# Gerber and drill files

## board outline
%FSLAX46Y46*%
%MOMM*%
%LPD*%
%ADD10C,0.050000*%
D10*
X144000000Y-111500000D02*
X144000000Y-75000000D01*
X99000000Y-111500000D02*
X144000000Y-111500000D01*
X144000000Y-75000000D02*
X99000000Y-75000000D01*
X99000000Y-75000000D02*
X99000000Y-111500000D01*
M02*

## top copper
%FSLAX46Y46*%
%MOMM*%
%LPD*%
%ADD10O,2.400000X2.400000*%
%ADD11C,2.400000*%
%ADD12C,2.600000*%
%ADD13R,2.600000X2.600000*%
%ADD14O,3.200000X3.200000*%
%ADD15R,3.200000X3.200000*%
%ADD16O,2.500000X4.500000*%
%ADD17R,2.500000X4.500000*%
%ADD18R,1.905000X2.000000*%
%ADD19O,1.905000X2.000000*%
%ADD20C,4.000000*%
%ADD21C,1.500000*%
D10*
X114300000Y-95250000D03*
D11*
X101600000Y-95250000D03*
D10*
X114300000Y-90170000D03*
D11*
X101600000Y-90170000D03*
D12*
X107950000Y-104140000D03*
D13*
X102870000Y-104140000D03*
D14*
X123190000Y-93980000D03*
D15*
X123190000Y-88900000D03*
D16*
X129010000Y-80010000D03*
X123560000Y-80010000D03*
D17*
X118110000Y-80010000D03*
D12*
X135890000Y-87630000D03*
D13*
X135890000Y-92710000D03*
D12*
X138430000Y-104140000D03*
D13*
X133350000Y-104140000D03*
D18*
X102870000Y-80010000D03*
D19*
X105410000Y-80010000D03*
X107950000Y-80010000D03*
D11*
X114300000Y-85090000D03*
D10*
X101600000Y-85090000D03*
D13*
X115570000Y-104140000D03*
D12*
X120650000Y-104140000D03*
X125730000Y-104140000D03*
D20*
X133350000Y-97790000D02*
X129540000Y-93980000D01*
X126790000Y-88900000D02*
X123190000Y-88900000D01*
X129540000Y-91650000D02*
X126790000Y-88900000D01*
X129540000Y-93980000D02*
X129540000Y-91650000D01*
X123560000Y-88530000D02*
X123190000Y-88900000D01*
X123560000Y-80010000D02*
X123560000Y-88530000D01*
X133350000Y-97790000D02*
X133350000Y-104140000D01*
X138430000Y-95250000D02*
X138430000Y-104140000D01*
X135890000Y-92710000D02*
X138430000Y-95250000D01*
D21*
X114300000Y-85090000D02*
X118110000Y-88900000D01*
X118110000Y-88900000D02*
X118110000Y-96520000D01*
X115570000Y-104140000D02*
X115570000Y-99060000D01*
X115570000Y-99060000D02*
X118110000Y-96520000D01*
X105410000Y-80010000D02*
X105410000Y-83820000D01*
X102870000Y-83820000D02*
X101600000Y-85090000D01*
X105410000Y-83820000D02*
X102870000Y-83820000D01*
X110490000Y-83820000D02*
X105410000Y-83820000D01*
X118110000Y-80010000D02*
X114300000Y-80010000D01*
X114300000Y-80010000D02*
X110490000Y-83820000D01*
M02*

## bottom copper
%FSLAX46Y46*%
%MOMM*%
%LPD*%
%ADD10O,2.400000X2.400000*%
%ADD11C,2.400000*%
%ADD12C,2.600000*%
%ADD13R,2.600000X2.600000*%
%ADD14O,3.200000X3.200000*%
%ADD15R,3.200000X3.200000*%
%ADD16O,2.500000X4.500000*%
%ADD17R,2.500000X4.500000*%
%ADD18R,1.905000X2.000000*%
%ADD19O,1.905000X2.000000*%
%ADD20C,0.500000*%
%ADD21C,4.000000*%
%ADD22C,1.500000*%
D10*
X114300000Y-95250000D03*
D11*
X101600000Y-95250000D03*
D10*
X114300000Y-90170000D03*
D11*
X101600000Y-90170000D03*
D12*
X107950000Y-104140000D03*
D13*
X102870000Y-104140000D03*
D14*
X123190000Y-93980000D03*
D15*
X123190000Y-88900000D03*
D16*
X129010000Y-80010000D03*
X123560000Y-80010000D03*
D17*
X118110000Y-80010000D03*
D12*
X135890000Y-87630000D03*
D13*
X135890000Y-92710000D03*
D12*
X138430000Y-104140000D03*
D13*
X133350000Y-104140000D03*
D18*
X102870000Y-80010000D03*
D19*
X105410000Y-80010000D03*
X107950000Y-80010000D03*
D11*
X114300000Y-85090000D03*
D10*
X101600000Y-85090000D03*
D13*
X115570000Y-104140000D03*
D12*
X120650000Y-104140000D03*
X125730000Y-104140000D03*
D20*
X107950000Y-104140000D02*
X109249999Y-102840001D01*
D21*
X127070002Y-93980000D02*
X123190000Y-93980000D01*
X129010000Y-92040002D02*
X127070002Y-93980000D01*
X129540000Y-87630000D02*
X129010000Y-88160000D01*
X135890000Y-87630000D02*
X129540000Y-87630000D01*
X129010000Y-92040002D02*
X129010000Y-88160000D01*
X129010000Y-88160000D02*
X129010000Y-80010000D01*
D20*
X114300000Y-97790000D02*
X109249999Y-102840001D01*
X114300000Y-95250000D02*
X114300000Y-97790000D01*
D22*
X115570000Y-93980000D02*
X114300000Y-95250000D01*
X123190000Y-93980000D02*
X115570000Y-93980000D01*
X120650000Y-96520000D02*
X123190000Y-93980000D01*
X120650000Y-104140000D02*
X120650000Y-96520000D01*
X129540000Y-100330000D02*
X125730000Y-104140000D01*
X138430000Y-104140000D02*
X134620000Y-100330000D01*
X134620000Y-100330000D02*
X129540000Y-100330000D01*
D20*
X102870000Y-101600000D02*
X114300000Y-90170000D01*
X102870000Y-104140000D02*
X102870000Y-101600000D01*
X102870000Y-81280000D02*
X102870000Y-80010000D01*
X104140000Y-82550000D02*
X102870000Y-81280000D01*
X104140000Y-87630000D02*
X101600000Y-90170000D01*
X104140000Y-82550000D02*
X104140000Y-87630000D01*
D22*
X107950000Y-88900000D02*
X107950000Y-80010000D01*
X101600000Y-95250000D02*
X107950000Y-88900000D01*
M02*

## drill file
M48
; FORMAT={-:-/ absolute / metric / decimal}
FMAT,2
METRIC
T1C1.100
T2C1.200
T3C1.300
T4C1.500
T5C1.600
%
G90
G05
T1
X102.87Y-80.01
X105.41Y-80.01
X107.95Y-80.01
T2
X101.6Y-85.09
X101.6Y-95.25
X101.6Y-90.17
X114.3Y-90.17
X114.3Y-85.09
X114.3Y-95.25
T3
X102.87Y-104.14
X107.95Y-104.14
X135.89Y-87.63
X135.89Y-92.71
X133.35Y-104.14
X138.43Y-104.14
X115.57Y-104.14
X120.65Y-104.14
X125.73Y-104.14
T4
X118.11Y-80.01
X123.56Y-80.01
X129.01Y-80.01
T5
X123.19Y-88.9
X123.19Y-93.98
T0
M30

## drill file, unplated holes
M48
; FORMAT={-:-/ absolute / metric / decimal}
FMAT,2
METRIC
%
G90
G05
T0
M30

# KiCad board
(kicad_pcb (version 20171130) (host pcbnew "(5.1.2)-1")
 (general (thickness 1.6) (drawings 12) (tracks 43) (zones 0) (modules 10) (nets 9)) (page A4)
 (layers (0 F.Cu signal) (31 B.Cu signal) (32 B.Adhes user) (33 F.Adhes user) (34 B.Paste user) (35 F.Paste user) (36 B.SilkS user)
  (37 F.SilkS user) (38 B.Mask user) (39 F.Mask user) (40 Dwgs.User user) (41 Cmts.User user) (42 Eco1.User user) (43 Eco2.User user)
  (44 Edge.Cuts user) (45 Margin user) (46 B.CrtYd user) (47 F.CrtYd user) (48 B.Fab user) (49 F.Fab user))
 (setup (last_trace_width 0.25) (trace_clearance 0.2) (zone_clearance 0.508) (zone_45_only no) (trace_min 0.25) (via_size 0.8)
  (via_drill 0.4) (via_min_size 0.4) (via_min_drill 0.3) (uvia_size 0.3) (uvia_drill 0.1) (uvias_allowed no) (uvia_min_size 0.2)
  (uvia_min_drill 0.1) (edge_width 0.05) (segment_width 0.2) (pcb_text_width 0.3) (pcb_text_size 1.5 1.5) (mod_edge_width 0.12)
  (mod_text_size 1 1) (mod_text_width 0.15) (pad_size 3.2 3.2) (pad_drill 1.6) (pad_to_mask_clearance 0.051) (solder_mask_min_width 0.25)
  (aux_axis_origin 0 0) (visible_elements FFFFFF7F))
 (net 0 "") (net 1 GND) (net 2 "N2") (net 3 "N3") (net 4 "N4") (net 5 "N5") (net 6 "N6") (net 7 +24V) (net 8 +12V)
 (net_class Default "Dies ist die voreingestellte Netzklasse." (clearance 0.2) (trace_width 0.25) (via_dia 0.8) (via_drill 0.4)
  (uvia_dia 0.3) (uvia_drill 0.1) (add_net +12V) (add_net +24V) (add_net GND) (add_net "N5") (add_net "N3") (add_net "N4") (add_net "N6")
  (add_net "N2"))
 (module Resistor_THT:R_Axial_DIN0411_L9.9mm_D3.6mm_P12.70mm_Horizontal (layer F.Cu) (at 101.6 95.25)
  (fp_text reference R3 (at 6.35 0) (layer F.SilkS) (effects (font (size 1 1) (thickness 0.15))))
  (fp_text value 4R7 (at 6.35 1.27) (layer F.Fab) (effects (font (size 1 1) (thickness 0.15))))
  (pad 2 thru_hole oval (at 12.7 0) (size 2.4 2.4) (drill 1.2) (layers *.Cu *.Mask) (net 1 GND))
  (pad 1 thru_hole circle (at 0 0) (size 2.4 2.4) (drill 1.2) (layers *.Cu *.Mask) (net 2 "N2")))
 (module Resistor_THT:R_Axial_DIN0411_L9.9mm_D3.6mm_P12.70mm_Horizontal (layer F.Cu) (at 101.6 90.17)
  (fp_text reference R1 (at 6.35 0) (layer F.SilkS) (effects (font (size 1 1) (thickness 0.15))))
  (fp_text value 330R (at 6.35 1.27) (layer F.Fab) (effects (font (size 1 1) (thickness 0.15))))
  (pad 2 thru_hole oval (at 12.7 0) (size 2.4 2.4) (drill 1.2) (layers *.Cu *.Mask) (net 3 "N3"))
  (pad 1 thru_hole circle (at 0 0) (size 2.4 2.4) (drill 1.2) (layers *.Cu *.Mask) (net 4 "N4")))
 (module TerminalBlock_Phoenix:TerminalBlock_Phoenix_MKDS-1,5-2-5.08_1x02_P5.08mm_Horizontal (layer F.Cu) (at 102.87 104.14)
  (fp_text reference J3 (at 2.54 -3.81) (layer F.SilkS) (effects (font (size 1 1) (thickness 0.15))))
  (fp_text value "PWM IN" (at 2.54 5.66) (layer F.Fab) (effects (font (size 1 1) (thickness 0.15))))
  (pad 2 thru_hole circle (at 5.08 0) (size 2.6 2.6) (drill 1.3) (layers *.Cu *.Mask) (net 1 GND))
  (pad 1 thru_hole rect (at 0 0) (size 2.6 2.6) (drill 1.3) (layers *.Cu *.Mask) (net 3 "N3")))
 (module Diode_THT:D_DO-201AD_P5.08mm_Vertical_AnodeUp (layer F.Cu) (at 123.19 88.9 270)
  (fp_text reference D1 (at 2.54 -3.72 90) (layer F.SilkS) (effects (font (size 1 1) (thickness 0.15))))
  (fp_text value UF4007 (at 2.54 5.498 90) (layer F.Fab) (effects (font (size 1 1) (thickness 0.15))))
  (pad 2 thru_hole oval (at 5.08 0 270) (size 3.2 3.2) (drill 1.6) (layers *.Cu *.Mask) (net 1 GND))
  (pad 1 thru_hole rect (at 0 0 270) (size 3.2 3.2) (drill 1.6) (layers *.Cu *.Mask) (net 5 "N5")))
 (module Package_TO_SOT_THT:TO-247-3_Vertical (layer F.Cu) (at 118.11 80.01)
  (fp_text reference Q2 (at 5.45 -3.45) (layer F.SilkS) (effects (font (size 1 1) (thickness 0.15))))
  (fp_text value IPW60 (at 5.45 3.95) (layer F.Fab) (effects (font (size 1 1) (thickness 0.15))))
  (pad 3 thru_hole oval (at 10.9 0) (size 2.5 4.5) (drill 1.5) (layers *.Cu *.Mask) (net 1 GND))
  (pad 2 thru_hole oval (at 5.45 0) (size 2.5 4.5) (drill 1.5) (layers *.Cu *.Mask) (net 5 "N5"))
  (pad 1 thru_hole rect (at 0 0) (size 2.5 4.5) (drill 1.5) (layers *.Cu *.Mask) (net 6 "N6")))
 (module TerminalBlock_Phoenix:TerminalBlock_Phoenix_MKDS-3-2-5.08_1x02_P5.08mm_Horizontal (layer F.Cu) (at 135.89 92.71 90)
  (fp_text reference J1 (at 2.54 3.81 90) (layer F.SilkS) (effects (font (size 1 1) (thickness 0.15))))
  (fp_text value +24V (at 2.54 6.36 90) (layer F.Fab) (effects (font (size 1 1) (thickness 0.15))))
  (pad 2 thru_hole circle (at 5.08 0 90) (size 2.6 2.6) (drill 1.3) (layers *.Cu *.Mask) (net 1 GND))
  (pad 1 thru_hole rect (at 0 0 90) (size 2.6 2.6) (drill 1.3) (layers *.Cu *.Mask) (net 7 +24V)))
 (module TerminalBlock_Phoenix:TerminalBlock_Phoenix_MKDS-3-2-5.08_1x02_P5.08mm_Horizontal (layer F.Cu) (at 133.35 104.14)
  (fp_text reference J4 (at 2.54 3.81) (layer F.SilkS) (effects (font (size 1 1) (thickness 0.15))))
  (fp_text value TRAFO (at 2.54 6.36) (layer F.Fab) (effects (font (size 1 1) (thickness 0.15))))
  (pad 2 thru_hole circle (at 5.08 0) (size 2.6 2.6) (drill 1.3) (layers *.Cu *.Mask) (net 7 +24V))
  (pad 1 thru_hole rect (at 0 0) (size 2.6 2.6) (drill 1.3) (layers *.Cu *.Mask) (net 5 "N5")))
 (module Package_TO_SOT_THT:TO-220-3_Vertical (layer F.Cu) (at 102.87 80.01)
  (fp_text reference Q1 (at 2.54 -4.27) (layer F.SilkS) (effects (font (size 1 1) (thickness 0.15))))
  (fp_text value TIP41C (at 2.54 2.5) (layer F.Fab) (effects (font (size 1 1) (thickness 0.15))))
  (pad 1 thru_hole rect (at 0 0) (size 1.905 2) (drill 1.1) (layers *.Cu *.Mask) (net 4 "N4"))
  (pad 2 thru_hole oval (at 2.54 0) (size 1.905 2) (drill 1.1) (layers *.Cu *.Mask) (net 6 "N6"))
  (pad 3 thru_hole oval (at 5.08 0) (size 1.905 2) (drill 1.1) (layers *.Cu *.Mask) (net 2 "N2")))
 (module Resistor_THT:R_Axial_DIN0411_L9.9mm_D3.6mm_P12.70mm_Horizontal (layer F.Cu) (at 114.3 85.09 180)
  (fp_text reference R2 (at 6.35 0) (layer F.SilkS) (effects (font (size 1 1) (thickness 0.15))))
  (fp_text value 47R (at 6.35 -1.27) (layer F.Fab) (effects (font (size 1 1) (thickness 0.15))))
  (pad 1 thru_hole circle (at 0 0 180) (size 2.4 2.4) (drill 1.2) (layers *.Cu *.Mask) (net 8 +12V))
  (pad 2 thru_hole oval (at 12.7 0 180) (size 2.4 2.4) (drill 1.2) (layers *.Cu *.Mask) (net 6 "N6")))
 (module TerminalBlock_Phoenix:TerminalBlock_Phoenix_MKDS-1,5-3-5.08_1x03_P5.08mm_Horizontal (layer F.Cu) (at 115.57 104.14)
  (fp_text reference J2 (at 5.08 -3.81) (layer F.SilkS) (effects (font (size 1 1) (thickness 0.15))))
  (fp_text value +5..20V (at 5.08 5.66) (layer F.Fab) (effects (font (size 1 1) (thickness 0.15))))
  (pad 1 thru_hole rect (at 0 0) (size 2.6 2.6) (drill 1.3) (layers *.Cu *.Mask) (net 8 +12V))
  (pad 2 thru_hole circle (at 5.08 0) (size 2.6 2.6) (drill 1.3) (layers *.Cu *.Mask) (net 1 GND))
  (pad 3 thru_hole circle (at 10.16 0) (size 2.6 2.6) (drill 1.3) (layers *.Cu *.Mask) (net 7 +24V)))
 (gr_line (start 144 111.5) (end 144 75) (layer Edge.Cuts) (width 0.05))
 (gr_line (start 99 111.5) (end 144 111.5) (layer Edge.Cuts) (width 0.05))
 (gr_line (start 144 75) (end 99 75) (layer Edge.Cuts) (width 0.05))
 (gr_line (start 99 75) (end 99 111.5) (layer Edge.Cuts) (width 0.05))
 (segment (start 133.35 97.79) (end 129.54 93.98) (width 4) (layer F.Cu) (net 5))
 (segment (start 126.79 88.9) (end 123.19 88.9) (width 4) (layer F.Cu) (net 5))
 (segment (start 129.54 91.65) (end 126.79 88.9) (width 4) (layer F.Cu) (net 5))
 (segment (start 129.54 93.98) (end 129.54 91.65) (width 4) (layer F.Cu) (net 5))
 (segment (start 123.56 88.53) (end 123.19 88.9) (width 4) (layer F.Cu) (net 5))
 (segment (start 123.56 80.01) (end 123.56 88.53) (width 4) (layer F.Cu) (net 5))
 (segment (start 133.35 97.79) (end 133.35 104.14) (width 4) (layer F.Cu) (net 5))
 (segment (start 107.95 104.14) (end 109.249999 102.840001) (width 0.5) (layer B.Cu) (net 1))
 (segment (start 127.070002 93.98) (end 123.19 93.98) (width 4) (layer B.Cu) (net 1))
 (segment (start 129.01 92.040002) (end 127.070002 93.98) (width 4) (layer B.Cu) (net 1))
 (segment (start 129.54 87.63) (end 129.01 88.16) (width 4) (layer B.Cu) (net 1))
 (segment (start 135.89 87.63) (end 129.54 87.63) (width 4) (layer B.Cu) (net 1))
 (segment (start 129.01 92.040002) (end 129.01 88.16) (width 4) (layer B.Cu) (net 1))
 (segment (start 129.01 88.16) (end 129.01 80.01) (width 4) (layer B.Cu) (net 1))
 (segment (start 114.3 97.79) (end 109.249999 102.840001) (width 0.5) (layer B.Cu) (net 1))
 (segment (start 114.3 95.25) (end 114.3 97.79) (width 0.5) (layer B.Cu) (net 1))
 (segment (start 115.57 93.98) (end 114.3 95.25) (width 1.5) (layer B.Cu) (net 1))
 (segment (start 123.19 93.98) (end 115.57 93.98) (width 1.5) (layer B.Cu) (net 1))
 (segment (start 120.65 96.52) (end 123.19 93.98) (width 1.5) (layer B.Cu) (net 1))
 (segment (start 120.65 104.14) (end 120.65 96.52) (width 1.5) (layer B.Cu) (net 1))
 (segment (start 138.43 95.25) (end 138.43 104.14) (width 4) (layer F.Cu) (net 7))
 (segment (start 135.89 92.71) (end 138.43 95.25) (width 4) (layer F.Cu) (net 7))
 (segment (start 129.54 100.33) (end 125.73 104.14) (width 1.5) (layer B.Cu) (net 7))
 (segment (start 138.43 104.14) (end 134.62 100.33) (width 1.5) (layer B.Cu) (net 7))
 (segment (start 134.62 100.33) (end 129.54 100.33) (width 1.5) (layer B.Cu) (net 7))
 (segment (start 114.3 85.09) (end 118.11 88.9) (width 1.5) (layer F.Cu) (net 8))
 (segment (start 118.11 88.9) (end 118.11 96.52) (width 1.5) (layer F.Cu) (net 8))
 (segment (start 115.57 104.14) (end 115.57 99.06) (width 1.5) (layer F.Cu) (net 8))
 (segment (start 115.57 99.06) (end 118.11 96.52) (width 1.5) (layer F.Cu) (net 8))
 (segment (start 102.87 101.6) (end 114.3 90.17) (width 0.5) (layer B.Cu) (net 3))
 (segment (start 102.87 104.14) (end 102.87 101.6) (width 0.5) (layer B.Cu) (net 3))
 (segment (start 102.87 81.28) (end 102.87 80.01) (width 0.5) (layer B.Cu) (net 4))
 (segment (start 104.14 82.55) (end 102.87 81.28) (width 0.5) (layer B.Cu) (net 4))
 (segment (start 104.14 87.63) (end 101.6 90.17) (width 0.5) (layer B.Cu) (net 4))
 (segment (start 104.14 82.55) (end 104.14 87.63) (width 0.5) (layer B.Cu) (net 4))
 (segment (start 105.41 80.01) (end 105.41 83.82) (width 1.5) (layer F.Cu) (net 6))
 (segment (start 102.87 83.82) (end 101.6 85.09) (width 1.5) (layer F.Cu) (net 6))
 (segment (start 105.41 83.82) (end 102.87 83.82) (width 1.5) (layer F.Cu) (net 6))
 (segment (start 110.49 83.82) (end 105.41 83.82) (width 1.5) (layer F.Cu) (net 6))
 (segment (start 118.11 80.01) (end 114.3 80.01) (width 1.5) (layer F.Cu) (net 6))
 (segment (start 114.3 80.01) (end 110.49 83.82) (width 1.5) (layer F.Cu) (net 6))
 (segment (start 107.95 88.9) (end 107.95 80.01) (width 1.5) (layer B.Cu) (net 2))
 (segment (start 101.6 95.25) (end 107.95 88.9) (width 1.5) (layer B.Cu) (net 2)))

